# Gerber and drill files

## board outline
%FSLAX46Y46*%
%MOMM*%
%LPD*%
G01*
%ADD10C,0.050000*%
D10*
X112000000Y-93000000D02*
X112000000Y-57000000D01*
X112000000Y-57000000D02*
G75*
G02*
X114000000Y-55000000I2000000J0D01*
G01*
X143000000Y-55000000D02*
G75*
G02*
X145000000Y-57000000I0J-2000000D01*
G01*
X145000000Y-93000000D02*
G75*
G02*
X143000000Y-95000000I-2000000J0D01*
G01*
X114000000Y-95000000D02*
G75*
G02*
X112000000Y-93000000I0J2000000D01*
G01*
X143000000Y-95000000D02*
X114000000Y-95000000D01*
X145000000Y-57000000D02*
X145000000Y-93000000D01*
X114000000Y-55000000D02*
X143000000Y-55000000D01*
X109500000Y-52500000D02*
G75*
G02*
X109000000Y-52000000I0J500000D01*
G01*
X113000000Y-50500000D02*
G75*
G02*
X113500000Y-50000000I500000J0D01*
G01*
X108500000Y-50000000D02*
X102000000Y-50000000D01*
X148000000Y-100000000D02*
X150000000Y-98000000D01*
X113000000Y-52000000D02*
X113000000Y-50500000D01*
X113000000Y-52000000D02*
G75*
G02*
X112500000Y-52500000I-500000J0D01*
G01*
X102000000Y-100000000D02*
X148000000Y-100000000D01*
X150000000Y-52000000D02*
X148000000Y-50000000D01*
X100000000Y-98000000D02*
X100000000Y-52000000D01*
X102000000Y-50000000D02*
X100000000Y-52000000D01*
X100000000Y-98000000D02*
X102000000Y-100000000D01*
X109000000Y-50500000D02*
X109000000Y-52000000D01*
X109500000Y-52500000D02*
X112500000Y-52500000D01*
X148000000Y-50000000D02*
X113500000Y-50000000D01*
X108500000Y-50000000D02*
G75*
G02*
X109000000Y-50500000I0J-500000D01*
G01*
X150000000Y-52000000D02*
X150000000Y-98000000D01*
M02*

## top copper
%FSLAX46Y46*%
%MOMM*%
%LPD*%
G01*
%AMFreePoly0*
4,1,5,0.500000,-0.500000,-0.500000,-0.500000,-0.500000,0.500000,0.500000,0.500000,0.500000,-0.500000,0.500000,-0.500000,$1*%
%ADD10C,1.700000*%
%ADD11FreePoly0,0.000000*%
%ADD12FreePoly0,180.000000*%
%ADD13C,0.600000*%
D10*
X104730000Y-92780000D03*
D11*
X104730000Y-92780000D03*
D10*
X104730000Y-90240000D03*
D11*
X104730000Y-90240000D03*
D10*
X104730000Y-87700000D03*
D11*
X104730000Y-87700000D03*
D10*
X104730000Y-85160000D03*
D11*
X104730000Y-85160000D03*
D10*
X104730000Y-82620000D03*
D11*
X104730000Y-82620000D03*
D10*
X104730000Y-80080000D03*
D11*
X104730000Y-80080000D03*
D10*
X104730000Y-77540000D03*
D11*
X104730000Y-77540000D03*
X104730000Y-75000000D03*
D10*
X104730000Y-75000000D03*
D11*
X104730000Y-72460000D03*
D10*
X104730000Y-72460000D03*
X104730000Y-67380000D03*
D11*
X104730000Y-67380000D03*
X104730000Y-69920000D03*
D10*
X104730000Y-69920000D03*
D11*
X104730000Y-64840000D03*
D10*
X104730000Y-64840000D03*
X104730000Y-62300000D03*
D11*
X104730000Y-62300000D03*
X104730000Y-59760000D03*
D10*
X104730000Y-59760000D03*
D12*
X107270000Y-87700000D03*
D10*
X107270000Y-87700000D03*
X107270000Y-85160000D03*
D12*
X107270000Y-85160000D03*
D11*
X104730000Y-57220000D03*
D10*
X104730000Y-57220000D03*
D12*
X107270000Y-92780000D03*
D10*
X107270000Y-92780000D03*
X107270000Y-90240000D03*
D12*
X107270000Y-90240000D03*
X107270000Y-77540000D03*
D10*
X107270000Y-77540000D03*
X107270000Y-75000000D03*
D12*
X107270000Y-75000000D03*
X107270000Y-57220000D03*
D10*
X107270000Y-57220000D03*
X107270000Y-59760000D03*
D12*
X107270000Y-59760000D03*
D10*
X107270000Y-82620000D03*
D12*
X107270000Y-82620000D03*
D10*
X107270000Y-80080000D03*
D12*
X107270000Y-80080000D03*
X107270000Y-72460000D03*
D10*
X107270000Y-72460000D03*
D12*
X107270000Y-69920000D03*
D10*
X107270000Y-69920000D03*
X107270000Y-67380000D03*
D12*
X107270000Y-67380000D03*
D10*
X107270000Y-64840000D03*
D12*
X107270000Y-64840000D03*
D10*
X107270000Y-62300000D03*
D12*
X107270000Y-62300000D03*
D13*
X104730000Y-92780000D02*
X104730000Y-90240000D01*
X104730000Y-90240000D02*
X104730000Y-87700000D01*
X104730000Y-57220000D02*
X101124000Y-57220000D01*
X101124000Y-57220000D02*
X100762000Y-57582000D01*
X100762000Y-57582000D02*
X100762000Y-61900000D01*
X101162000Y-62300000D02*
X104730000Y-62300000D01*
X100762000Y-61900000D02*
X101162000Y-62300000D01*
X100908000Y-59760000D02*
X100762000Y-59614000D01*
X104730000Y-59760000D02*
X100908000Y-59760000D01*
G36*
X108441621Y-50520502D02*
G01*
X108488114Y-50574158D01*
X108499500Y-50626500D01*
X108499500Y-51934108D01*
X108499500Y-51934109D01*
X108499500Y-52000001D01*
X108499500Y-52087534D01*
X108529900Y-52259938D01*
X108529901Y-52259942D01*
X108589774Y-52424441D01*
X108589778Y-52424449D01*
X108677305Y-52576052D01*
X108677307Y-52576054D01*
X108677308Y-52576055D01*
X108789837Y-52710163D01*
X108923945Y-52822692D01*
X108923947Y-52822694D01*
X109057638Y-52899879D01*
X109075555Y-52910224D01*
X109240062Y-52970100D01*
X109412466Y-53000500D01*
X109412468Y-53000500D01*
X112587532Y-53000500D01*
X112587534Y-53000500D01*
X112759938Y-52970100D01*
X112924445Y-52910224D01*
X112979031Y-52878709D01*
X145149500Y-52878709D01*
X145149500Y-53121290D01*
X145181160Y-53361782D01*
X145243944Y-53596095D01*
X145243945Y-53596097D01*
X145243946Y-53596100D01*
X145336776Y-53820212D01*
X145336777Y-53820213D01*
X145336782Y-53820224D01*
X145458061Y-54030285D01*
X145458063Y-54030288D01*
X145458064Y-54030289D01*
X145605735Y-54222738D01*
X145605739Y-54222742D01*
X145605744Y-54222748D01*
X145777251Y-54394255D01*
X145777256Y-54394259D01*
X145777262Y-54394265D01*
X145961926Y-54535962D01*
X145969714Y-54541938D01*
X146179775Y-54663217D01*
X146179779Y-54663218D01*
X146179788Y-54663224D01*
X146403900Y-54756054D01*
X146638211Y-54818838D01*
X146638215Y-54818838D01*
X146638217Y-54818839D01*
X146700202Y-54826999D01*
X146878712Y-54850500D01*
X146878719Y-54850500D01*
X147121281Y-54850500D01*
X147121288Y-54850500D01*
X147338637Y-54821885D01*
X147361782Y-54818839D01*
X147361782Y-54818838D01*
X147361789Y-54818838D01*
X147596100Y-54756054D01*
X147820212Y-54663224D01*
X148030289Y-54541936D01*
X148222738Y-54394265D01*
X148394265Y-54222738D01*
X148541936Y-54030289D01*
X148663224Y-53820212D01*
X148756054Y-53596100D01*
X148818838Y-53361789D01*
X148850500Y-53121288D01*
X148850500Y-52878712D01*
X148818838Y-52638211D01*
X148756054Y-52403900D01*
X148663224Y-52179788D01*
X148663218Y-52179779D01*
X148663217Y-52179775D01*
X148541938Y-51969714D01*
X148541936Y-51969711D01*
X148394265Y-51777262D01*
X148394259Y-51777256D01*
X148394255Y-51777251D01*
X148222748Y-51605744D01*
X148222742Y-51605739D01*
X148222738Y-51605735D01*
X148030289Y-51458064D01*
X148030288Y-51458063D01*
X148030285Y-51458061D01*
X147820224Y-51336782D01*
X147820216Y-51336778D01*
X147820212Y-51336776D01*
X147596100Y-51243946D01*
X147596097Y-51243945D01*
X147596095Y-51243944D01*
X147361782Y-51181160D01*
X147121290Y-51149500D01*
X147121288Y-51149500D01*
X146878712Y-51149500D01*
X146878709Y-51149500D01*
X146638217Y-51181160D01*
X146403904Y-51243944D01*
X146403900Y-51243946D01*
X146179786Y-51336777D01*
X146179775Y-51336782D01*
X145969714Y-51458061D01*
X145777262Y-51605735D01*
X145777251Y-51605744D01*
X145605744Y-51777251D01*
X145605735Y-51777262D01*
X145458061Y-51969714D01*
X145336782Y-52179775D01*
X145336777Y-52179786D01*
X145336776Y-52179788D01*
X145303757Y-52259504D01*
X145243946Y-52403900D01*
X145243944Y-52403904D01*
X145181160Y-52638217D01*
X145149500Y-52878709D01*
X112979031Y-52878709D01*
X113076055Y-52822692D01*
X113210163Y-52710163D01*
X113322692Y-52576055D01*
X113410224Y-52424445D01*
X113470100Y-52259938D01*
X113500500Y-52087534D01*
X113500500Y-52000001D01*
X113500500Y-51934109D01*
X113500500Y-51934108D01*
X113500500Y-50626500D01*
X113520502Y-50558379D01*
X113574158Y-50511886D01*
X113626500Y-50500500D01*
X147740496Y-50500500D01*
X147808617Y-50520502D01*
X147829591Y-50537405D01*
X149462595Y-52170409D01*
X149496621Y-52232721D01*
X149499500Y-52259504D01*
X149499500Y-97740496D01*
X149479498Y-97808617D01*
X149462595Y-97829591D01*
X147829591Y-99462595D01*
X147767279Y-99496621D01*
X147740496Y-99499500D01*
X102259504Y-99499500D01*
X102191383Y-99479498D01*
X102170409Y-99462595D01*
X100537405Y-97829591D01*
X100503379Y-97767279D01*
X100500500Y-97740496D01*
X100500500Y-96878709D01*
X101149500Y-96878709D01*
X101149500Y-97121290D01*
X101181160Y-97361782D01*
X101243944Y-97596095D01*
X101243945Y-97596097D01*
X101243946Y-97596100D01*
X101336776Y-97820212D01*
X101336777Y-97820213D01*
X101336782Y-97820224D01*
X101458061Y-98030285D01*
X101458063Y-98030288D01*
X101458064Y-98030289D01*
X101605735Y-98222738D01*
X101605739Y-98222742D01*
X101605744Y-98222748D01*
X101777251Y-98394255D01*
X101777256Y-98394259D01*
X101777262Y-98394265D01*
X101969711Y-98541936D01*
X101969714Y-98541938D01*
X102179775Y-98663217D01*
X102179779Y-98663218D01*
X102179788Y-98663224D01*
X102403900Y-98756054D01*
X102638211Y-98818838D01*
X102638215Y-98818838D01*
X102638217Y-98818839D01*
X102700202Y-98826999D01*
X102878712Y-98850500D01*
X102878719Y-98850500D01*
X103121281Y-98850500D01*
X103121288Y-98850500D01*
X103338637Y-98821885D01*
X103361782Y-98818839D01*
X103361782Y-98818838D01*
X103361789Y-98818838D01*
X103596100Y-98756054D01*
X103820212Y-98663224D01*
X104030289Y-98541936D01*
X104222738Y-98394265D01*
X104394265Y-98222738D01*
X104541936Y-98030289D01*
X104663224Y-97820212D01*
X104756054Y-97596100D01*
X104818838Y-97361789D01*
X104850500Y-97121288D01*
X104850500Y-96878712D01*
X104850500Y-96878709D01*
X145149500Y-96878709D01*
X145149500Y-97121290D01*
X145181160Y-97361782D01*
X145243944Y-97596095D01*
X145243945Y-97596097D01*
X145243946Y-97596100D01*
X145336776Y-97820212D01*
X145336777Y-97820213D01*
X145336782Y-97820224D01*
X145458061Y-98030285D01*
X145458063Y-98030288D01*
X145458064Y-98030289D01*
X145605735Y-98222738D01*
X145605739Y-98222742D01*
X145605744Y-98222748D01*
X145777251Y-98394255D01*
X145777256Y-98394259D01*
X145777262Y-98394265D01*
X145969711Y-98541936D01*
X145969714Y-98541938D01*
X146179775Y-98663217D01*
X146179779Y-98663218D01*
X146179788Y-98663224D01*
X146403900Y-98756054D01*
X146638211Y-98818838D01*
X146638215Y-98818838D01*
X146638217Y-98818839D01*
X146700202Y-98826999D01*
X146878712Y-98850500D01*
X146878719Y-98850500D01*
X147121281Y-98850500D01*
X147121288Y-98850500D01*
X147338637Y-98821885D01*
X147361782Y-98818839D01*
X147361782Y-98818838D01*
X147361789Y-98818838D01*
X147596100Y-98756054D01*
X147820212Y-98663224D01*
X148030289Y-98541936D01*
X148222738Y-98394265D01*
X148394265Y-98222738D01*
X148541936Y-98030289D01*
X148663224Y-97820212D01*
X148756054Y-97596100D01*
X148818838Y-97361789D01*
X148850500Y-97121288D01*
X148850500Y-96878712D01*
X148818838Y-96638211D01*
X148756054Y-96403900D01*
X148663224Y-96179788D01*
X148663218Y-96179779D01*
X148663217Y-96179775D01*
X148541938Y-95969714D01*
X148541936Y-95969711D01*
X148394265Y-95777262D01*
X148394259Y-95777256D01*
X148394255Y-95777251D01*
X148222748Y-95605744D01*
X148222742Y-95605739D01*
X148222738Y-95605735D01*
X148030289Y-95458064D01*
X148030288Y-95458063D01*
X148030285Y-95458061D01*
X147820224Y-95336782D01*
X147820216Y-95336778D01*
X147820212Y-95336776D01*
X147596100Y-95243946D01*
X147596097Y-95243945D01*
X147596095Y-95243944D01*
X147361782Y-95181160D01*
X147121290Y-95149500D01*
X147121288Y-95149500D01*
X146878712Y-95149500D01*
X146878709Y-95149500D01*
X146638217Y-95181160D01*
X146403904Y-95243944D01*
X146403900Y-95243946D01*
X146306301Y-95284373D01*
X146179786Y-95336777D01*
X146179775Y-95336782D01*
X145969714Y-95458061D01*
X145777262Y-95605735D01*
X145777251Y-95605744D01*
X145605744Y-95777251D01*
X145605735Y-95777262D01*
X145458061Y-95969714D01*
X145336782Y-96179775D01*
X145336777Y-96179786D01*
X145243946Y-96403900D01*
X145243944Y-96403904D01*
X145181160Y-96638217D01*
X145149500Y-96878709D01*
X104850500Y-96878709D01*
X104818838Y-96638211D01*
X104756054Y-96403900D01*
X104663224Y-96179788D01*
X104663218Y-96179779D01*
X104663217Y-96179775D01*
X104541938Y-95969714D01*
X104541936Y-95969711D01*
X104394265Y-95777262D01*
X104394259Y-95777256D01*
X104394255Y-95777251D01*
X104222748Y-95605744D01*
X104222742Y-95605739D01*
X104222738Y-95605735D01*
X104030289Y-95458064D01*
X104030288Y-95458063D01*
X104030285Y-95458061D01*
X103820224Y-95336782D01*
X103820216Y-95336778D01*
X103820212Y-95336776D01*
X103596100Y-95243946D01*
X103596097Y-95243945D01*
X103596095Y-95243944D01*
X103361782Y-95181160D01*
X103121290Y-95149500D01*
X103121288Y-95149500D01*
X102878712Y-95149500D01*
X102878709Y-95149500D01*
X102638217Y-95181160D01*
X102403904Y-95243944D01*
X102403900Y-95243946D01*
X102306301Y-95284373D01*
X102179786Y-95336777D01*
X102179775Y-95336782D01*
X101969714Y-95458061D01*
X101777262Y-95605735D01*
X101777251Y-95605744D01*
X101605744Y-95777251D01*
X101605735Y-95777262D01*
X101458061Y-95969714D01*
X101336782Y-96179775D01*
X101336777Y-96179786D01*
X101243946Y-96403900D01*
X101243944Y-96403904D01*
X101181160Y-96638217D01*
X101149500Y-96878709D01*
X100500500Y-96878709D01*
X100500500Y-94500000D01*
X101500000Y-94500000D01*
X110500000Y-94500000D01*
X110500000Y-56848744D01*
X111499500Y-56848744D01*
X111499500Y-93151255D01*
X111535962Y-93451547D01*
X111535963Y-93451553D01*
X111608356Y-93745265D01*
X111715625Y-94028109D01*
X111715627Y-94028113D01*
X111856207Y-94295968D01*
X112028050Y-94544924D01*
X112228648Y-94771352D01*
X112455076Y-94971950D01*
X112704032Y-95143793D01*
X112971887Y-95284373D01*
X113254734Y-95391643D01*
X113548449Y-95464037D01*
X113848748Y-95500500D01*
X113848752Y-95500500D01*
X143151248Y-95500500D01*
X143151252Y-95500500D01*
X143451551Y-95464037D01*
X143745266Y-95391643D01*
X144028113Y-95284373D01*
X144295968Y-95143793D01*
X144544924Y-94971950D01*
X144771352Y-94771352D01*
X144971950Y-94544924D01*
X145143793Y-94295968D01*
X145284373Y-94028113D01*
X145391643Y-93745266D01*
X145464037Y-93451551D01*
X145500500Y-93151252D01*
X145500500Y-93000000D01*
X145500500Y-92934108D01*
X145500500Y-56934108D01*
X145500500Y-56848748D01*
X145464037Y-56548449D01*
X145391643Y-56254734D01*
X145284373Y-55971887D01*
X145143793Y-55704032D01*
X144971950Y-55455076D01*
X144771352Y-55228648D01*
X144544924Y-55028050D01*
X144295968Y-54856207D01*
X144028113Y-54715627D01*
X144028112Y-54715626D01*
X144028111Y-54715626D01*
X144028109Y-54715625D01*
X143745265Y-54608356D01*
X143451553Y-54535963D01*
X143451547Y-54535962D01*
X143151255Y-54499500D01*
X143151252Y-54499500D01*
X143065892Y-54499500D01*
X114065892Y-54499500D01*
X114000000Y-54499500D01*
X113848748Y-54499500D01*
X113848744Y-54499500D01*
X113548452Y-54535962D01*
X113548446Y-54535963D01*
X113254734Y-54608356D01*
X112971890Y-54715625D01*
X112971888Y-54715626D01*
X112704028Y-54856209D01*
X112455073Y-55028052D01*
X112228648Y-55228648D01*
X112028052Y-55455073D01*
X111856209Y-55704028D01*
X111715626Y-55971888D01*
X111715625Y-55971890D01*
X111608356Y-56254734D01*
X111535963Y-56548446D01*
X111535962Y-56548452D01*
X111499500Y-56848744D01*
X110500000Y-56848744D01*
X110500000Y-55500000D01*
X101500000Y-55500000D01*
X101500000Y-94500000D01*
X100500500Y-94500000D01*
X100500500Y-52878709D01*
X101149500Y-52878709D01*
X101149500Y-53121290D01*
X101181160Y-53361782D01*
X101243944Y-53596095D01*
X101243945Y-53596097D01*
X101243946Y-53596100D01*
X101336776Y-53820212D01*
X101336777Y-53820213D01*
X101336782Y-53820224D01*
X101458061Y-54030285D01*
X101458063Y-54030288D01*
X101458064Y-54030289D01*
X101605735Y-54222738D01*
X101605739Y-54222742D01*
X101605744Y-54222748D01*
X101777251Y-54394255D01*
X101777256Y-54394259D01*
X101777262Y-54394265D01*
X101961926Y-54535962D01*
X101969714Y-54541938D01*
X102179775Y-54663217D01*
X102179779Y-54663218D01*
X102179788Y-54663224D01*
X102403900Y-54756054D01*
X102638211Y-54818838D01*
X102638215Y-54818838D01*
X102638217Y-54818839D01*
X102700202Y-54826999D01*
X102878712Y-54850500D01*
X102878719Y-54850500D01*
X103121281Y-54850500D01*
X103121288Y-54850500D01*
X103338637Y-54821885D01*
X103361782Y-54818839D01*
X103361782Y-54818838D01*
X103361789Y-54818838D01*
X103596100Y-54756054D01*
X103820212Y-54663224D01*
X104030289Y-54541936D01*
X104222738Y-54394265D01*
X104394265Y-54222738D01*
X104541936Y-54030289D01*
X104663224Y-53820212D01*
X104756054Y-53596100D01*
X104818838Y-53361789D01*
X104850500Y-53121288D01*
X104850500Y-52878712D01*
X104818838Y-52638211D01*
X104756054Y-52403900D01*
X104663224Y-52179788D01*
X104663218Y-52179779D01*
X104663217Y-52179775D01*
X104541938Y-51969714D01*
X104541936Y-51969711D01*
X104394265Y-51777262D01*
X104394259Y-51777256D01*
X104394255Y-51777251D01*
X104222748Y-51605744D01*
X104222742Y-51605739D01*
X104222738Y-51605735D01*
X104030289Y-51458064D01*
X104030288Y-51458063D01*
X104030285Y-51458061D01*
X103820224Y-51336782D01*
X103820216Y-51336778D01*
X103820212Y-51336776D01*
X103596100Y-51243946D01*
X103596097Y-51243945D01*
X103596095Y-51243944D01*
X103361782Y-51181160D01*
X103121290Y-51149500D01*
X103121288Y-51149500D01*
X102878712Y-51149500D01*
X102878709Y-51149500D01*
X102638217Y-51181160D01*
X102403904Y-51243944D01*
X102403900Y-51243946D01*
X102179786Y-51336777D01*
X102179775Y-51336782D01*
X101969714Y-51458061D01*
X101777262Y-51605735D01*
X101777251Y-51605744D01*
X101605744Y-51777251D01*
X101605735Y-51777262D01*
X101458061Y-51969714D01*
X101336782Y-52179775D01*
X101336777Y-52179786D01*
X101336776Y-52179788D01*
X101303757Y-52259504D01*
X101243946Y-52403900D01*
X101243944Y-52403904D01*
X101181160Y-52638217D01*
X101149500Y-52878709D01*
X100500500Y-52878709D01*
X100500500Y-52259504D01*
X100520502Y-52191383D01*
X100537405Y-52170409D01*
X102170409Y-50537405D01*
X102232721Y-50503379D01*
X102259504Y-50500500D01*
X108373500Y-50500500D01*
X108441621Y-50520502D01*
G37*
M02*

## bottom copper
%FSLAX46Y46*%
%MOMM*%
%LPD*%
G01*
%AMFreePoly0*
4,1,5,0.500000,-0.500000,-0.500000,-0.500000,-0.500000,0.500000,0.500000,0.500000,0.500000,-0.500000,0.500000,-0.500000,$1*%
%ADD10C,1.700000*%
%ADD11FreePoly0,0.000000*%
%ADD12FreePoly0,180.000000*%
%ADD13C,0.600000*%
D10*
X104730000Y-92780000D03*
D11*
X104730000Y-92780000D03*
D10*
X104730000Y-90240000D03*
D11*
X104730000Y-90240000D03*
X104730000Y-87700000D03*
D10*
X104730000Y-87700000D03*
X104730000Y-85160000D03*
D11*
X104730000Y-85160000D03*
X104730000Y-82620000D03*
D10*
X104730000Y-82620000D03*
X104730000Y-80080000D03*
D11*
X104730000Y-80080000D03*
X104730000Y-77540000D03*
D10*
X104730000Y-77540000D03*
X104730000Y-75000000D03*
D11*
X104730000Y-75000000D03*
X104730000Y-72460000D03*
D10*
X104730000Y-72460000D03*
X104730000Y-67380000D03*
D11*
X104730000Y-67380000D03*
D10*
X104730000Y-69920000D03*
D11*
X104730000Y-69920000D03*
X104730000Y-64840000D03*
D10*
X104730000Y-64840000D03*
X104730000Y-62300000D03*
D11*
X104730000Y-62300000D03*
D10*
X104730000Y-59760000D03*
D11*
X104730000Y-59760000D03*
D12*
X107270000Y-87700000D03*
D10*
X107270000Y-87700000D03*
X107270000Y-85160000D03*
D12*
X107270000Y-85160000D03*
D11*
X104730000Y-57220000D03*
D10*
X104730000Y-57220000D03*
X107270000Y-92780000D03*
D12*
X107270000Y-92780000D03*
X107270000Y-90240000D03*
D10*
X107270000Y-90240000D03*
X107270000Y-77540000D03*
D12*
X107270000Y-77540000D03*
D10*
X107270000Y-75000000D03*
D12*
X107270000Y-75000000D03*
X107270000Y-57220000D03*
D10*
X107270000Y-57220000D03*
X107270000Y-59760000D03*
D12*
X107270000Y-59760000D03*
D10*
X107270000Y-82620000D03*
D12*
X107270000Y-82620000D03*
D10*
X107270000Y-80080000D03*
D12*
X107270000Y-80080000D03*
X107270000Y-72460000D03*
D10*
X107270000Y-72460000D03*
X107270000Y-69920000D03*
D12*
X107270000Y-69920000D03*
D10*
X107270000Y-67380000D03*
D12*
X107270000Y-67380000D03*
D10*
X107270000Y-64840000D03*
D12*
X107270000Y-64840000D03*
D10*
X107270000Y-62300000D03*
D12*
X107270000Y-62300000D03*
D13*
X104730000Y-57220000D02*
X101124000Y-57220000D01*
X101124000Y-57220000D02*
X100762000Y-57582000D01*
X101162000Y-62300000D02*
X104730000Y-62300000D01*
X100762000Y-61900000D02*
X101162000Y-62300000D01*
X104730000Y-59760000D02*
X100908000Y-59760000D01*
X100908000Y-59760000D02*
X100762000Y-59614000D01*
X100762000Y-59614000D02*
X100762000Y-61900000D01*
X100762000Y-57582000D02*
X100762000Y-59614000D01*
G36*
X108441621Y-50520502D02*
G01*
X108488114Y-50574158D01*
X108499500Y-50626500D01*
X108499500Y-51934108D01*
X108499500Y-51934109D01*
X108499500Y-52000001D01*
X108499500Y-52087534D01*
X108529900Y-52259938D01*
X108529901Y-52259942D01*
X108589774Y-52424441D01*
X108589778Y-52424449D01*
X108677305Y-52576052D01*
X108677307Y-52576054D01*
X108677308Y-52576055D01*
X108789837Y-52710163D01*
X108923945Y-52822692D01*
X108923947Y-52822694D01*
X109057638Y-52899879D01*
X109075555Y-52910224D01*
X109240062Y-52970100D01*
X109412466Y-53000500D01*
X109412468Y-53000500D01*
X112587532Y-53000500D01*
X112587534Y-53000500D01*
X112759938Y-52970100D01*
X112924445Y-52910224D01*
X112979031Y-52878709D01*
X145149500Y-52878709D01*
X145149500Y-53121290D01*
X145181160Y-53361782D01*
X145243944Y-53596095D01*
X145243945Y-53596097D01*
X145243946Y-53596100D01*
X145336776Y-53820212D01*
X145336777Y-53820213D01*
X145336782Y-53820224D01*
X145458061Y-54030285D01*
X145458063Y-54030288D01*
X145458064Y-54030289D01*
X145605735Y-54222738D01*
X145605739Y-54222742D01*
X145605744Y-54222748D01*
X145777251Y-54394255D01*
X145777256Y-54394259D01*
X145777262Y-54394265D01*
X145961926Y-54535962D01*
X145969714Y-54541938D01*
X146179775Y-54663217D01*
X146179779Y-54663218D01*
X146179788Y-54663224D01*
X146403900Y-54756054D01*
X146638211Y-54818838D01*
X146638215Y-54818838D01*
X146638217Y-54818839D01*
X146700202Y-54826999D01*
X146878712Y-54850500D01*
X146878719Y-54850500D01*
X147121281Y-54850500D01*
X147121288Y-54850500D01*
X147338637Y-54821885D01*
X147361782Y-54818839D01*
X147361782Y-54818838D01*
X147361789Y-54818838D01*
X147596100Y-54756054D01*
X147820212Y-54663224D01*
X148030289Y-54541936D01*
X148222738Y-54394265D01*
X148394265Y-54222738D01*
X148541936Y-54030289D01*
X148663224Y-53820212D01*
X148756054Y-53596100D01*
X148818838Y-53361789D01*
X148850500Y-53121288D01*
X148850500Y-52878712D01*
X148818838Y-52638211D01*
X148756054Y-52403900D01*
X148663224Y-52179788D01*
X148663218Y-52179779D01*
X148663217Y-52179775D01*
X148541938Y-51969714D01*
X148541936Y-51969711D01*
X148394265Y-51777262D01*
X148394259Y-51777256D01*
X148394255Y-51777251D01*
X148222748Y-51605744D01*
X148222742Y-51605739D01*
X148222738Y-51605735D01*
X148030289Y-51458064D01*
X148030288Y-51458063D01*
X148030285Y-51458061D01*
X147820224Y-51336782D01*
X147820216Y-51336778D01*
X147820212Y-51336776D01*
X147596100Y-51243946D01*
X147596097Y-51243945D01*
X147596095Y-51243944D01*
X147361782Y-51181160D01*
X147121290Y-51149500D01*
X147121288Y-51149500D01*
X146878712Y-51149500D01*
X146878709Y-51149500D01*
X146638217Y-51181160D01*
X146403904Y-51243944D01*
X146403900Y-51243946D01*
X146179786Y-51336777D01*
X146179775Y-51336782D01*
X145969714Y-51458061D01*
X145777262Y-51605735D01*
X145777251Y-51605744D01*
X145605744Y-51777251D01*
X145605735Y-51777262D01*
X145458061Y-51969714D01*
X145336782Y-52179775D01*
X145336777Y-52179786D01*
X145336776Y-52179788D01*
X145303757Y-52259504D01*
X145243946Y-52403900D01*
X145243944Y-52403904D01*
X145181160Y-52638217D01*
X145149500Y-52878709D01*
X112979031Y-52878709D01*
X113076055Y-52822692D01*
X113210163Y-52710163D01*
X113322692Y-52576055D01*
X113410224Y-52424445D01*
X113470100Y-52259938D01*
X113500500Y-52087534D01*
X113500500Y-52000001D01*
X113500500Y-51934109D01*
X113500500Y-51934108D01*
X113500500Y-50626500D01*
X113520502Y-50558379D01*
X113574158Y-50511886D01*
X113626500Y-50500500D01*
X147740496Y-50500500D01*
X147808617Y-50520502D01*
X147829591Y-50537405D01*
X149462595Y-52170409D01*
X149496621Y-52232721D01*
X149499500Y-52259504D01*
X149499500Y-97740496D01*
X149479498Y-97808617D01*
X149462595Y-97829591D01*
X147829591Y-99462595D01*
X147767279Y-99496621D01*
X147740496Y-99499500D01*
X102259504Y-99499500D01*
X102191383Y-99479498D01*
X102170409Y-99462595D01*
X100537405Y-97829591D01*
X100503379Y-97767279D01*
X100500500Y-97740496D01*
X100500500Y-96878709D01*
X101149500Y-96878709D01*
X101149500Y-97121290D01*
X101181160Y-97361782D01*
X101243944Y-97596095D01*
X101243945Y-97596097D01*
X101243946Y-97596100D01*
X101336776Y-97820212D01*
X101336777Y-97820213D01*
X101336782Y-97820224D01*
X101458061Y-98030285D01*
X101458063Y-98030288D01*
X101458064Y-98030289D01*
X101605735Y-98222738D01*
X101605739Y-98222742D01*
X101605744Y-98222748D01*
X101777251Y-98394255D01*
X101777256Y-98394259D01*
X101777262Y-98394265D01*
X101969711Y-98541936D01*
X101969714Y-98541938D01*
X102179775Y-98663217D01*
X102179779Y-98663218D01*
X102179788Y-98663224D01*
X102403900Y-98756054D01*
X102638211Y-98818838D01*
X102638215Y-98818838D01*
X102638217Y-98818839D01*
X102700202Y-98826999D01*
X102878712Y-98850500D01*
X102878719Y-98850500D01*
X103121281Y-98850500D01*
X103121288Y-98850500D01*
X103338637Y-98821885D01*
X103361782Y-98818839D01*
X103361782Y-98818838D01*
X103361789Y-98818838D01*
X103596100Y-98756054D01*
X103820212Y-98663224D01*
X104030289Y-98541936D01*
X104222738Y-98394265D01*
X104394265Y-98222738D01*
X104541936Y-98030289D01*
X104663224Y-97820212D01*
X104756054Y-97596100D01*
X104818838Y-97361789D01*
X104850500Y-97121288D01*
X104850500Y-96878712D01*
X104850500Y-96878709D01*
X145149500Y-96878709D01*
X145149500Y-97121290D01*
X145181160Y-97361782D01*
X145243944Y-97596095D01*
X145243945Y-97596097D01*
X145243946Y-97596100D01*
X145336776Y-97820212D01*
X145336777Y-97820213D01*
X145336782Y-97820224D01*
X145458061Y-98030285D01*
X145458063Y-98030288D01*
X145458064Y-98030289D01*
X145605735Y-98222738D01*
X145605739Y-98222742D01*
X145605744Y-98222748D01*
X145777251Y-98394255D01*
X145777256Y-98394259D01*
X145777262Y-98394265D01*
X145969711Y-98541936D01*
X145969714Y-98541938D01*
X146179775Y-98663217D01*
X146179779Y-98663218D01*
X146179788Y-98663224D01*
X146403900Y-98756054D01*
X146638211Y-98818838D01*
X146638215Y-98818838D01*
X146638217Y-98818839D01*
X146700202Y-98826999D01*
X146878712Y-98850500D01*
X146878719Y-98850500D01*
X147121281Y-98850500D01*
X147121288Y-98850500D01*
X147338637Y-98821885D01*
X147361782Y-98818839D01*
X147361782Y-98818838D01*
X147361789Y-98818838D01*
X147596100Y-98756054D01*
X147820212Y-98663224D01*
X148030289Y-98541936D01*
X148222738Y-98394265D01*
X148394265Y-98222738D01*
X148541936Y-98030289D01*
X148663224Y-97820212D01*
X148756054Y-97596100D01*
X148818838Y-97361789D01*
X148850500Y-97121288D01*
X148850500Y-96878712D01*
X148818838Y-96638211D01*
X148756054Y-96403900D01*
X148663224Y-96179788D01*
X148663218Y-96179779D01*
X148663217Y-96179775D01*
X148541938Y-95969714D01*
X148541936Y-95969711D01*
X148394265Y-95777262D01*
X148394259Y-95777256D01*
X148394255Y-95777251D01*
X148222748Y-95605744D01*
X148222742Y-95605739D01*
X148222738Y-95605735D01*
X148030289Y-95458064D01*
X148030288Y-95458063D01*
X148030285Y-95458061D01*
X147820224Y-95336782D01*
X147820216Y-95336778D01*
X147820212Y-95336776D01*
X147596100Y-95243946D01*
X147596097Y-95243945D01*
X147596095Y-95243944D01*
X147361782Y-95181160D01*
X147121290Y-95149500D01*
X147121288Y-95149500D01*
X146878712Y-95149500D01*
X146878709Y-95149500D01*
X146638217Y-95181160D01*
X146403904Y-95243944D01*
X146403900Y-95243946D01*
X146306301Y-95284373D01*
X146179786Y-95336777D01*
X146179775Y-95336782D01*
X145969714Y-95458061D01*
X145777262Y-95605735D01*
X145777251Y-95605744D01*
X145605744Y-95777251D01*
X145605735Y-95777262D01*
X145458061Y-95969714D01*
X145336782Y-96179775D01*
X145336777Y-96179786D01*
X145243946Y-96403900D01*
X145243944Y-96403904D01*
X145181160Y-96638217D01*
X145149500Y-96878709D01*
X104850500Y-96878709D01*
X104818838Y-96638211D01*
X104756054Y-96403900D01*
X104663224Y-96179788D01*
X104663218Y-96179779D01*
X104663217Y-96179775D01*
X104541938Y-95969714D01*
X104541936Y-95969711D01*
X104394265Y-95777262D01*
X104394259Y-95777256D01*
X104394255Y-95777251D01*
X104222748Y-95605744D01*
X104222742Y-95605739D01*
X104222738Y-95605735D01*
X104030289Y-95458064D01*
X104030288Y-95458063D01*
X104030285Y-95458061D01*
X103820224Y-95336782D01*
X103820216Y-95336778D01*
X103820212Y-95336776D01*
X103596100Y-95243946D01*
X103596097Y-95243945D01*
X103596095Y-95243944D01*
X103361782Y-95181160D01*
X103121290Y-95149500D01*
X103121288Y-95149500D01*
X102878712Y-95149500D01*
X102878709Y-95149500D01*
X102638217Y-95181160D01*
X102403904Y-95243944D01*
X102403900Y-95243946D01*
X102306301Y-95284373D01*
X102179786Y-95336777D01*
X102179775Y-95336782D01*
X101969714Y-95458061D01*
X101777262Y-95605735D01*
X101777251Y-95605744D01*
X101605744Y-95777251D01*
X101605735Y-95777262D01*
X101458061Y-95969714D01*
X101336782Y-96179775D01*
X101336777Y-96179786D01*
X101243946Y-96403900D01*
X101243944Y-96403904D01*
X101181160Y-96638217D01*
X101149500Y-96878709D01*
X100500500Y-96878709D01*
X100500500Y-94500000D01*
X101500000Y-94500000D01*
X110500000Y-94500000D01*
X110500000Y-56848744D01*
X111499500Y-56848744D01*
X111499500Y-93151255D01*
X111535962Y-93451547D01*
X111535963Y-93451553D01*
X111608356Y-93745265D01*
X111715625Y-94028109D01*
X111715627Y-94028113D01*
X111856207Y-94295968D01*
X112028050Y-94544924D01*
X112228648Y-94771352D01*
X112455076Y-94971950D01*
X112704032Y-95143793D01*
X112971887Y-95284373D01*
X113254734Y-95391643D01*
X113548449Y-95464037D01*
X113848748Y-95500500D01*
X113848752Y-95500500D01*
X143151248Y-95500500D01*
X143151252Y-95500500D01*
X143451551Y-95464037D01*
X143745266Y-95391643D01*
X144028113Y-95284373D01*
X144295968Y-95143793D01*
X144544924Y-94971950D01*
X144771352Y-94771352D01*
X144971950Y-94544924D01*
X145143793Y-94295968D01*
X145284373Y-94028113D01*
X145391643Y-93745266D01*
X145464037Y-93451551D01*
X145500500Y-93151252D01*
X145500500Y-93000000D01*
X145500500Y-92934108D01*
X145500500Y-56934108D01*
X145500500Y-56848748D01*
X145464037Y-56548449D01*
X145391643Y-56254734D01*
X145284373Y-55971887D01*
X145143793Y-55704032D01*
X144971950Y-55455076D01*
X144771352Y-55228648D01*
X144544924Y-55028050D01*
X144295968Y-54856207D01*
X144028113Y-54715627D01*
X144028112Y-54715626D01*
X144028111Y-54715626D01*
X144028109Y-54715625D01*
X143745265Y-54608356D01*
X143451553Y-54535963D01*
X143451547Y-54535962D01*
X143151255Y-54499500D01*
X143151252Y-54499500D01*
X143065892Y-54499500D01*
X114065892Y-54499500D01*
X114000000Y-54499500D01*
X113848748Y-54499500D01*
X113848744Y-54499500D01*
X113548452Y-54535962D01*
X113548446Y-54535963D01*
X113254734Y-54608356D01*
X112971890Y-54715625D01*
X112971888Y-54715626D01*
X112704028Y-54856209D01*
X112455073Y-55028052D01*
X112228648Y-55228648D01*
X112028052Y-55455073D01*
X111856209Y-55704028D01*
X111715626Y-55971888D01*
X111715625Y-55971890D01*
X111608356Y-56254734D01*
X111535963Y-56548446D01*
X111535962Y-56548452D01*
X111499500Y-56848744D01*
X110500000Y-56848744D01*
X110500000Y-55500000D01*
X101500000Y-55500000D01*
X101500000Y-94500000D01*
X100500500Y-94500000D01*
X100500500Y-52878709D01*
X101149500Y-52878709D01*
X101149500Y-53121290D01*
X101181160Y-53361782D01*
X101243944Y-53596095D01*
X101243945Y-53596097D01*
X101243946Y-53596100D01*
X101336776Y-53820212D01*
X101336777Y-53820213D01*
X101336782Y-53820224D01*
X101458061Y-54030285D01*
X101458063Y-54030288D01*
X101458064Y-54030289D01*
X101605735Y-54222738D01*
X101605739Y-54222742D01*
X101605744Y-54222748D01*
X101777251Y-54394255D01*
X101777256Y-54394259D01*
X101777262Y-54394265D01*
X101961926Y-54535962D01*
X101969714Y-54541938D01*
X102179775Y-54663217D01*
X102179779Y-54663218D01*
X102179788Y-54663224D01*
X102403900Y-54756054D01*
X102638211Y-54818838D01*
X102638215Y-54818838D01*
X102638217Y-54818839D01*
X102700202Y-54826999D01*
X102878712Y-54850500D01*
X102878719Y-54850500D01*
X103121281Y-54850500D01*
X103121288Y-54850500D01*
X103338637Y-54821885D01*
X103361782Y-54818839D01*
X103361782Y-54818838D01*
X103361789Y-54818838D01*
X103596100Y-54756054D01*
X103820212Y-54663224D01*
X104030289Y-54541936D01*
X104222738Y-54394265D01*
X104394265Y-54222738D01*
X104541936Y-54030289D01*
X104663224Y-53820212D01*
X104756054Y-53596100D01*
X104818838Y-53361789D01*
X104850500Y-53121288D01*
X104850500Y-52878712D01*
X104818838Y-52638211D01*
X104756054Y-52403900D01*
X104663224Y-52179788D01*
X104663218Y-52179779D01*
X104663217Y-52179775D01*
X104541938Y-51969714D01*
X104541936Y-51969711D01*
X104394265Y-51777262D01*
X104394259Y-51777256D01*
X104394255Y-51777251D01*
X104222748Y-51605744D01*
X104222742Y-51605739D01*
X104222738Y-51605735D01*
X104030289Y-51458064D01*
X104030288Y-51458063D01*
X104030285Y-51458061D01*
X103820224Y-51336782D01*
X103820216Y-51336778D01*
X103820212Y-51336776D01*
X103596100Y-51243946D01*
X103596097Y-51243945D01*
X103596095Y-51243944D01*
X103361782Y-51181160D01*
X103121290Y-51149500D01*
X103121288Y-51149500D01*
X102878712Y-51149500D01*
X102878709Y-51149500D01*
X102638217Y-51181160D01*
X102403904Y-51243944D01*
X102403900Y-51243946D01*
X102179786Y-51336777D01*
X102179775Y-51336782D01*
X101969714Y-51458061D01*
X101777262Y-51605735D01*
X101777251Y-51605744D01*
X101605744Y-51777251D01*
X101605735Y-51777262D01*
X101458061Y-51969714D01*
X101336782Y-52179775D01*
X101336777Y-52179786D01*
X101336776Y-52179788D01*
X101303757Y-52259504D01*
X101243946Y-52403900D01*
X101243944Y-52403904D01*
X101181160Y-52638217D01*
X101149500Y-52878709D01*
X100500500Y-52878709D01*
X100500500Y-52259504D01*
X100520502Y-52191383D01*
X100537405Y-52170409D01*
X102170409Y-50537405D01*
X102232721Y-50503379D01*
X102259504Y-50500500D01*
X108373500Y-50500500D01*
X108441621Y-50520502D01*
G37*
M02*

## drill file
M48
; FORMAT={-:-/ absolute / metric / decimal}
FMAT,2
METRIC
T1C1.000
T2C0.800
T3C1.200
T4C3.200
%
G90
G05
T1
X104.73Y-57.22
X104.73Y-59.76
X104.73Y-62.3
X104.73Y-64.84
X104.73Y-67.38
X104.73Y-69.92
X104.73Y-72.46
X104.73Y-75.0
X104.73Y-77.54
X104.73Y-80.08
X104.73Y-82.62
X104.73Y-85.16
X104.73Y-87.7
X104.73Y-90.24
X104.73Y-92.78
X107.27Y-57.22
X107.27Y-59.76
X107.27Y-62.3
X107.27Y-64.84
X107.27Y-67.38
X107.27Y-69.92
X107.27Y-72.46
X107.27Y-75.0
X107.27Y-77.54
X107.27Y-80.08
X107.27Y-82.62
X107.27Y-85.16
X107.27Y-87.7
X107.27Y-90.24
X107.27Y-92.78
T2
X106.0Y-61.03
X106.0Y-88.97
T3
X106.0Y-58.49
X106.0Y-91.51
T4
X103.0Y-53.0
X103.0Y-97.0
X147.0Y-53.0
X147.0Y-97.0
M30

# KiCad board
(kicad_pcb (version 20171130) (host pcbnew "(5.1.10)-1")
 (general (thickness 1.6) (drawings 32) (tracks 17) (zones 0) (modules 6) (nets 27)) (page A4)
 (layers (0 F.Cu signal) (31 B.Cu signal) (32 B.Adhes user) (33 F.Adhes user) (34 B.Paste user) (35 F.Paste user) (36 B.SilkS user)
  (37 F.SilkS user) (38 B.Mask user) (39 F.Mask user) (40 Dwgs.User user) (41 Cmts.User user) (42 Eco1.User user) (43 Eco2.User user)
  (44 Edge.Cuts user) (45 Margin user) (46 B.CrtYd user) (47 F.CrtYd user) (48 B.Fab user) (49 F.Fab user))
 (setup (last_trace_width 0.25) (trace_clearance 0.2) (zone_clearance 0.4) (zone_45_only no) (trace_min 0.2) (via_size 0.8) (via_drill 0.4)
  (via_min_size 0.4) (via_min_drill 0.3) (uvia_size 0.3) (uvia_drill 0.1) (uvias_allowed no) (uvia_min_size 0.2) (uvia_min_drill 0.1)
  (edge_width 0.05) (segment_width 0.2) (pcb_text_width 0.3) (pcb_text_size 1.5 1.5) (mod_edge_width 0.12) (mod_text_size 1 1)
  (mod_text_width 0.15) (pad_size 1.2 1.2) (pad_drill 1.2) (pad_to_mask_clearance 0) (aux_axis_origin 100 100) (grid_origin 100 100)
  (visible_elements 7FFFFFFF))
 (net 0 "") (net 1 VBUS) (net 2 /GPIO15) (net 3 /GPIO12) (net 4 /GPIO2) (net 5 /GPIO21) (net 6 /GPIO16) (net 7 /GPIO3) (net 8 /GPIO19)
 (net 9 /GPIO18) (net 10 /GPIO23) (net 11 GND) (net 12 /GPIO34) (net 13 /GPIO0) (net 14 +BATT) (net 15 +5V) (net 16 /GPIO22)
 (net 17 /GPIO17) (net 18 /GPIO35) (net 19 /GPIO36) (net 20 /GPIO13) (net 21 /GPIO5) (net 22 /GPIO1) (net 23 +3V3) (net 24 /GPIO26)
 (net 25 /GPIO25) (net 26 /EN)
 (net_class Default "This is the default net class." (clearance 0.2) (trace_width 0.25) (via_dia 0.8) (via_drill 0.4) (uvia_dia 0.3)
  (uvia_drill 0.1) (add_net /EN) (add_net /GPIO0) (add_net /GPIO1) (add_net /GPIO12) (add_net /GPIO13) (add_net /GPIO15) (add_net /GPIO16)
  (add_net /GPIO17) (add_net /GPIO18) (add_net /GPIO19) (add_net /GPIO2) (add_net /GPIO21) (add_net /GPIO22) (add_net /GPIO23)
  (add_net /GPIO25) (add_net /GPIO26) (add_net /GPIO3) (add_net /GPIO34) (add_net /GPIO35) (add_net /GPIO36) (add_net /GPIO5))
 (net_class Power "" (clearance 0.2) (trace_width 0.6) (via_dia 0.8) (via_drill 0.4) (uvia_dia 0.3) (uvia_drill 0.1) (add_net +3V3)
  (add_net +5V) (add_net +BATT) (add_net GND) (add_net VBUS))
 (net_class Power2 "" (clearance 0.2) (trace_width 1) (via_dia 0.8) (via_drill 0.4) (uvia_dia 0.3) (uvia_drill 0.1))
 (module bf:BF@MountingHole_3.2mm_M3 (layer F.Cu) (at 147 97)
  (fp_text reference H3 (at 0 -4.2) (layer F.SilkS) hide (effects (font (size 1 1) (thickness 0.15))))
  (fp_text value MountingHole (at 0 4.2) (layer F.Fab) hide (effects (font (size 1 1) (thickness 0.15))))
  (pad "" np_thru_hole circle (at 0 0) (size 3.2 3.2) (drill 3.2) (layers *.Cu *.Mask)))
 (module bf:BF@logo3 (layer F.Cu) (at 130 97.5)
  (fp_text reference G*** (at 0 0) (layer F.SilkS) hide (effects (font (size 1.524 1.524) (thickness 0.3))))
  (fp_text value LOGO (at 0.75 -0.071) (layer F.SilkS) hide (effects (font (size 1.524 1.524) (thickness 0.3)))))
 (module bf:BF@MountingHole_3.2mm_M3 (layer F.Cu) (at 103 97)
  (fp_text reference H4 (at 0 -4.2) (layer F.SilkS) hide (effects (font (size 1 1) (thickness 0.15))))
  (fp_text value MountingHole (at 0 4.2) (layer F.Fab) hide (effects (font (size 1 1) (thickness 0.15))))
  (pad "" np_thru_hole circle (at 0 0) (size 3.2 3.2) (drill 3.2) (layers *.Cu *.Mask)))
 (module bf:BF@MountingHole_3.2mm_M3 (layer F.Cu) (at 147 53)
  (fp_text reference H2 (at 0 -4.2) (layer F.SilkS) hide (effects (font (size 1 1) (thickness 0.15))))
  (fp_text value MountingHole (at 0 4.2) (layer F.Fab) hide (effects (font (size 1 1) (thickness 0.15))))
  (pad "" np_thru_hole circle (at 0 0) (size 3.2 3.2) (drill 3.2) (layers *.Cu *.Mask)))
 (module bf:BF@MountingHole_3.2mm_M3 (layer F.Cu) (at 103 53)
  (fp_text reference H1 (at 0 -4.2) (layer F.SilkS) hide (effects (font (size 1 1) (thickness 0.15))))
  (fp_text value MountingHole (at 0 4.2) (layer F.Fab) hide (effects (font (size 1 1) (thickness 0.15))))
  (pad "" np_thru_hole circle (at 0 0) (size 3.2 3.2) (drill 3.2) (layers *.Cu *.Mask)))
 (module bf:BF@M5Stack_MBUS (layer F.Cu) (at 106 75)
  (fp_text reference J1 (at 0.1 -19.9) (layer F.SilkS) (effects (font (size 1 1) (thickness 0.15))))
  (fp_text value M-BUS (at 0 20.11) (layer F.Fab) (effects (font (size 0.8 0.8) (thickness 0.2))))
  (pad 30 thru_hole circle (at -1.27 17.78) (size 1.7 1.7) (drill 1) (layers *.Cu *.Mask) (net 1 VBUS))
  (pad 30 smd custom (at -1.27 17.78) (size 1 1) (layers B.Cu B.Mask) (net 1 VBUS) (zone_connect 0)
   (options (clearance outline) (anchor rect)) (primitives))
  (pad 30 smd custom (at -1.27 17.78) (size 1 1) (layers F.Cu F.Mask) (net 1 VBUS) (zone_connect 0)
   (options (clearance outline) (anchor rect)) (primitives))
  (pad 28 thru_hole circle (at -1.27 15.24) (size 1.7 1.7) (drill 1) (layers *.Cu *.Mask) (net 1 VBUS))
  (pad 28 smd custom (at -1.27 15.24) (size 1 1) (layers B.Cu B.Mask) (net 1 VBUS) (zone_connect 0)
   (options (clearance outline) (anchor rect)) (primitives))
  (pad 28 smd custom (at -1.27 15.24) (size 1 1) (layers F.Cu F.Mask) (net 1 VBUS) (zone_connect 0)
   (options (clearance outline) (anchor rect)) (primitives))
  (pad 26 smd custom (at -1.27 12.7) (size 1 1) (layers B.Cu B.Mask) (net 1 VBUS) (zone_connect 0)
   (options (clearance outline) (anchor rect)) (primitives))
  (pad 26 thru_hole circle (at -1.27 12.7) (size 1.7 1.7) (drill 1) (layers *.Cu *.Mask) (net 1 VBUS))
  (pad 26 smd custom (at -1.27 12.7) (size 1 1) (layers F.Cu F.Mask) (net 1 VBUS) (zone_connect 0)
   (options (clearance outline) (anchor rect)) (primitives))
  (pad 24 thru_hole circle (at -1.27 10.16) (size 1.7 1.7) (drill 1) (layers *.Cu *.Mask) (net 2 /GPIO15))
  (pad 24 smd custom (at -1.27 10.16) (size 1 1) (layers B.Cu B.Mask) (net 2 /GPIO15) (zone_connect 0)
   (options (clearance outline) (anchor rect)) (primitives))
  (pad 24 smd custom (at -1.27 10.16) (size 1 1) (layers F.Cu F.Mask) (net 2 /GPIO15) (zone_connect 0)
   (options (clearance outline) (anchor rect)) (primitives))
  (pad 22 smd custom (at -1.27 7.62) (size 1 1) (layers B.Cu B.Mask) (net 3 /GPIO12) (zone_connect 0)
   (options (clearance outline) (anchor rect)) (primitives))
  (pad 22 thru_hole circle (at -1.27 7.62) (size 1.7 1.7) (drill 1) (layers *.Cu *.Mask) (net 3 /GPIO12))
  (pad 22 smd custom (at -1.27 7.62) (size 1 1) (layers F.Cu F.Mask) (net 3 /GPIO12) (zone_connect 0)
   (options (clearance outline) (anchor rect)) (primitives))
  (pad 20 thru_hole circle (at -1.27 5.08) (size 1.7 1.7) (drill 1) (layers *.Cu *.Mask) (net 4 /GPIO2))
  (pad 20 smd custom (at -1.27 5.08) (size 1 1) (layers F.Cu F.Mask) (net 4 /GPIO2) (zone_connect 0)
   (options (clearance outline) (anchor rect)) (primitives))
  (pad 20 smd custom (at -1.27 5.08) (size 1 1) (layers B.Cu B.Mask) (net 4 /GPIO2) (zone_connect 0)
   (options (clearance outline) (anchor rect)) (primitives))
  (pad 18 smd custom (at -1.27 2.54) (size 1 1) (layers B.Cu B.Mask) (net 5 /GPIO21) (zone_connect 0)
   (options (clearance outline) (anchor rect)) (primitives))
  (pad 18 thru_hole circle (at -1.27 2.54) (size 1.7 1.7) (drill 1) (layers *.Cu *.Mask) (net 5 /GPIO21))
  (pad 18 smd custom (at -1.27 2.54) (size 1 1) (layers F.Cu F.Mask) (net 5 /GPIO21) (zone_connect 0)
   (options (clearance outline) (anchor rect)) (primitives))
  (pad 16 smd custom (at -1.27 0) (size 1 1) (layers F.Cu F.Mask) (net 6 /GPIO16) (zone_connect 0)
   (options (clearance outline) (anchor rect)) (primitives))
  (pad 16 thru_hole circle (at -1.27 0) (size 1.7 1.7) (drill 1) (layers *.Cu *.Mask) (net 6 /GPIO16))
  (pad 16 smd custom (at -1.27 0) (size 1 1) (layers B.Cu B.Mask) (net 6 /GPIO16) (zone_connect 0)
   (options (clearance outline) (anchor rect)) (primitives))
  (pad 14 smd custom (at -1.27 -2.54) (size 1 1) (layers B.Cu B.Mask) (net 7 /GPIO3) (zone_connect 0)
   (options (clearance outline) (anchor rect)) (primitives))
  (pad 14 smd custom (at -1.27 -2.54) (size 1 1) (layers F.Cu F.Mask) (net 7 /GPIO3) (zone_connect 0)
   (options (clearance outline) (anchor rect)) (primitives))
  (pad 14 thru_hole circle (at -1.27 -2.54) (size 1.7 1.7) (drill 1) (layers *.Cu *.Mask) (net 7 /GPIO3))
  (pad 10 thru_hole circle (at -1.27 -7.62) (size 1.7 1.7) (drill 1) (layers *.Cu *.Mask) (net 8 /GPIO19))
  (pad 10 smd custom (at -1.27 -7.62) (size 1 1) (layers B.Cu B.Mask) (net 8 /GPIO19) (zone_connect 0)
   (options (clearance outline) (anchor rect)) (primitives))
  (pad 10 smd custom (at -1.27 -7.62) (size 1 1) (layers F.Cu F.Mask) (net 8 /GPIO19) (zone_connect 0)
   (options (clearance outline) (anchor rect)) (primitives))
  (pad 12 smd custom (at -1.27 -5.08) (size 1 1) (layers F.Cu F.Mask) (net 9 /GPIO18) (zone_connect 0)
   (options (clearance outline) (anchor rect)) (primitives))
  (pad 12 thru_hole circle (at -1.27 -5.08) (size 1.7 1.7) (drill 1) (layers *.Cu *.Mask) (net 9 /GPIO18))
  (pad 12 smd custom (at -1.27 -5.08) (size 1 1) (layers B.Cu B.Mask) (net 9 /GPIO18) (zone_connect 0)
   (options (clearance outline) (anchor rect)) (primitives))
  (pad 8 smd custom (at -1.27 -10.16) (size 1 1) (layers B.Cu B.Mask) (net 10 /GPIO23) (zone_connect 0)
   (options (clearance outline) (anchor rect)) (primitives))
  (pad 8 smd custom (at -1.27 -10.16) (size 1 1) (layers F.Cu F.Mask) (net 10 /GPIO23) (zone_connect 0)
   (options (clearance outline) (anchor rect)) (primitives))
  (pad 8 thru_hole circle (at -1.27 -10.16) (size 1.7 1.7) (drill 1) (layers *.Cu *.Mask) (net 10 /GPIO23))
  (pad 6 thru_hole circle (at -1.27 -12.7) (size 1.7 1.7) (drill 1) (layers *.Cu *.Mask) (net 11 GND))
  (pad 6 smd custom (at -1.27 -12.7) (size 1 1) (layers F.Cu F.Mask) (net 11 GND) (zone_connect 0)
   (options (clearance outline) (anchor rect)) (primitives))
  (pad 6 smd custom (at -1.27 -12.7) (size 1 1) (layers B.Cu B.Mask) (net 11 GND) (zone_connect 0)
   (options (clearance outline) (anchor rect)) (primitives))
  (pad 4 smd custom (at -1.27 -15.24) (size 1 1) (layers F.Cu F.Mask) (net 11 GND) (zone_connect 0)
   (options (clearance outline) (anchor rect)) (primitives))
  (pad 4 thru_hole circle (at -1.27 -15.24) (size 1.7 1.7) (drill 1) (layers *.Cu *.Mask) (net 11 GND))
  (pad 4 smd custom (at -1.27 -15.24) (size 1 1) (layers B.Cu B.Mask) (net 11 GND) (zone_connect 0)
   (options (clearance outline) (anchor rect)) (primitives))
  (pad 25 smd custom (at 1.27 12.7 180) (size 1 1) (layers B.Cu B.Mask) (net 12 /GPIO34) (zone_connect 0)
   (options (clearance outline) (anchor rect)) (primitives))
  (pad 25 smd custom (at 1.27 12.7 180) (size 1 1) (layers F.Cu F.Mask) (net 12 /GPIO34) (zone_connect 0)
   (options (clearance outline) (anchor rect)) (primitives))
  (pad 25 thru_hole circle (at 1.27 12.7 180) (size 1.7 1.7) (drill 1) (layers *.Cu *.Mask) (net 12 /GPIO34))
  (pad 23 thru_hole circle (at 1.27 10.16 180) (size 1.7 1.7) (drill 1) (layers *.Cu *.Mask) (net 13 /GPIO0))
  (pad 23 smd custom (at 1.27 10.16 180) (size 1 1) (layers F.Cu F.Mask) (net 13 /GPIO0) (zone_connect 0)
   (options (clearance outline) (anchor rect)) (primitives))
  (pad 23 smd custom (at 1.27 10.16 180) (size 1 1) (layers B.Cu B.Mask) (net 13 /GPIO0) (zone_connect 0)
   (options (clearance outline) (anchor rect)) (primitives))
  (pad 2 smd custom (at -1.27 -17.78) (size 1 1) (layers F.Cu F.Mask) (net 11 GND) (zone_connect 0)
   (options (clearance outline) (anchor rect)) (primitives))
  (pad 2 smd custom (at -1.27 -17.78) (size 1 1) (layers B.Cu B.Mask) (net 11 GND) (zone_connect 0)
   (options (clearance outline) (anchor rect)) (primitives))
  (pad 2 thru_hole circle (at -1.27 -17.78) (size 1.7 1.7) (drill 1) (layers *.Cu *.Mask) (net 11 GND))
  (pad 29 smd custom (at 1.27 17.78 180) (size 1 1) (layers F.Cu F.Mask) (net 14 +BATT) (zone_connect 0)
   (options (clearance outline) (anchor rect)) (primitives))
  (pad 29 thru_hole circle (at 1.27 17.78 180) (size 1.7 1.7) (drill 1) (layers *.Cu *.Mask) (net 14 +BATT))
  (pad 29 smd custom (at 1.27 17.78 180) (size 1 1) (layers B.Cu B.Mask) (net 14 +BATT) (zone_connect 0)
   (options (clearance outline) (anchor rect)) (primitives))
  (pad 27 smd custom (at 1.27 15.24 180) (size 1 1) (layers B.Cu B.Mask) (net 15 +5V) (zone_connect 0)
   (options (clearance outline) (anchor rect)) (primitives))
  (pad 27 thru_hole circle (at 1.27 15.24 180) (size 1.7 1.7) (drill 1) (layers *.Cu *.Mask) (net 15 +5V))
  (pad 27 smd custom (at 1.27 15.24 180) (size 1 1) (layers F.Cu F.Mask) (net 15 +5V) (zone_connect 0)
   (options (clearance outline) (anchor rect)) (primitives))
  (pad 17 smd custom (at 1.27 2.54 180) (size 1 1) (layers F.Cu F.Mask) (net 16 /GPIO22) (zone_connect 0)
   (options (clearance outline) (anchor rect)) (primitives))
  (pad 17 thru_hole circle (at 1.27 2.54 180) (size 1.7 1.7) (drill 1) (layers *.Cu *.Mask) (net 16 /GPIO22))
  (pad 17 smd custom (at 1.27 2.54 180) (size 1 1) (layers B.Cu B.Mask) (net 16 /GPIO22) (zone_connect 0)
   (options (clearance outline) (anchor rect)) (primitives))
  (pad 15 thru_hole circle (at 1.27 0 180) (size 1.7 1.7) (drill 1) (layers *.Cu *.Mask) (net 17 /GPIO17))
  (pad 15 smd custom (at 1.27 0 180) (size 1 1) (layers B.Cu B.Mask) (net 17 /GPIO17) (zone_connect 0)
   (options (clearance outline) (anchor rect)) (primitives))
  (pad 15 smd custom (at 1.27 0 180) (size 1 1) (layers F.Cu F.Mask) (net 17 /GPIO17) (zone_connect 0)
   (options (clearance outline) (anchor rect)) (primitives))
  (pad "" np_thru_hole circle (at 0 13.97 180) (size 0.8 0.8) (drill 0.8) (layers *.Cu *.Mask))
  (pad 1 smd custom (at 1.27 -17.78 180) (size 1 1) (layers F.Cu F.Mask) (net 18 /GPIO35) (zone_connect 0)
   (options (clearance outline) (anchor rect)) (primitives))
  (pad 1 smd custom (at 1.27 -17.78 180) (size 1 1) (layers B.Cu B.Mask) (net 18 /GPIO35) (zone_connect 0)
   (options (clearance outline) (anchor rect)) (primitives))
  (pad "" np_thru_hole circle (at 0 16.51 180) (size 1.2 1.2) (drill 1.2) (layers *.Cu *.Mask))
  (pad "" np_thru_hole circle (at 0 -13.97 180) (size 0.8 0.8) (drill 0.8) (layers *.Cu *.Mask))
  (pad 1 thru_hole circle (at 1.27 -17.78 180) (size 1.7 1.7) (drill 1) (layers *.Cu *.Mask) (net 18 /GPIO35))
  (pad "" np_thru_hole circle (at 0 -16.51 180) (size 1.2 1.2) (drill 1.2) (layers *.Cu *.Mask))
  (pad 3 thru_hole circle (at 1.27 -15.24 180) (size 1.7 1.7) (drill 1) (layers *.Cu *.Mask) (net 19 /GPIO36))
  (pad 3 smd custom (at 1.27 -15.24 180) (size 1 1) (layers B.Cu B.Mask) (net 19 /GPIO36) (zone_connect 0)
   (options (clearance outline) (anchor rect)) (primitives))
  (pad 3 smd custom (at 1.27 -15.24 180) (size 1 1) (layers F.Cu F.Mask) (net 19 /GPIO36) (zone_connect 0)
   (options (clearance outline) (anchor rect)) (primitives))
  (pad 21 thru_hole circle (at 1.27 7.62 180) (size 1.7 1.7) (drill 1) (layers *.Cu *.Mask) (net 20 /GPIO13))
  (pad 21 smd custom (at 1.27 7.62 180) (size 1 1) (layers B.Cu B.Mask) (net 20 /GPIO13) (zone_connect 0)
   (options (clearance outline) (anchor rect)) (primitives))
  (pad 21 smd custom (at 1.27 7.62 180) (size 1 1) (layers F.Cu F.Mask) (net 20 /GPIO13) (zone_connect 0)
   (options (clearance outline) (anchor rect)) (primitives))
  (pad 19 thru_hole circle (at 1.27 5.08 180) (size 1.7 1.7) (drill 1) (layers *.Cu *.Mask) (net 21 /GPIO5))
  (pad 19 smd custom (at 1.27 5.08 180) (size 1 1) (layers F.Cu F.Mask) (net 21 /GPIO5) (zone_connect 0)
   (options (clearance outline) (anchor rect)) (primitives))
  (pad 19 smd custom (at 1.27 5.08 180) (size 1 1) (layers B.Cu B.Mask) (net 21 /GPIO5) (zone_connect 0)
   (options (clearance outline) (anchor rect)) (primitives))
  (pad 13 smd custom (at 1.27 -2.54 180) (size 1 1) (layers F.Cu F.Mask) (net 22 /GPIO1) (zone_connect 0)
   (options (clearance outline) (anchor rect)) (primitives))
  (pad 13 smd custom (at 1.27 -2.54 180) (size 1 1) (layers B.Cu B.Mask) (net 22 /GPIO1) (zone_connect 0)
   (options (clearance outline) (anchor rect)) (primitives))
  (pad 13 thru_hole circle (at 1.27 -2.54 180) (size 1.7 1.7) (drill 1) (layers *.Cu *.Mask) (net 22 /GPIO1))
  (pad 11 smd custom (at 1.27 -5.08 180) (size 1 1) (layers F.Cu F.Mask) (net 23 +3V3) (zone_connect 0)
   (options (clearance outline) (anchor rect)) (primitives))
  (pad 11 thru_hole circle (at 1.27 -5.08 180) (size 1.7 1.7) (drill 1) (layers *.Cu *.Mask) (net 23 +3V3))
  (pad 11 smd custom (at 1.27 -5.08 180) (size 1 1) (layers B.Cu B.Mask) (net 23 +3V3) (zone_connect 0)
   (options (clearance outline) (anchor rect)) (primitives))
  (pad 9 thru_hole circle (at 1.27 -7.62 180) (size 1.7 1.7) (drill 1) (layers *.Cu *.Mask) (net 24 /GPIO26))
  (pad 9 smd custom (at 1.27 -7.62 180) (size 1 1) (layers B.Cu B.Mask) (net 24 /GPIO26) (zone_connect 0)
   (options (clearance outline) (anchor rect)) (primitives))
  (pad 9 smd custom (at 1.27 -7.62 180) (size 1 1) (layers F.Cu F.Mask) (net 24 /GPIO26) (zone_connect 0)
   (options (clearance outline) (anchor rect)) (primitives))
  (pad 7 thru_hole circle (at 1.27 -10.16 180) (size 1.7 1.7) (drill 1) (layers *.Cu *.Mask) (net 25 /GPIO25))
  (pad 7 smd custom (at 1.27 -10.16 180) (size 1 1) (layers F.Cu F.Mask) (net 25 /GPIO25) (zone_connect 0)
   (options (clearance outline) (anchor rect)) (primitives))
  (pad 7 smd custom (at 1.27 -10.16 180) (size 1 1) (layers B.Cu B.Mask) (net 25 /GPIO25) (zone_connect 0)
   (options (clearance outline) (anchor rect)) (primitives))
  (pad 5 thru_hole circle (at 1.27 -12.7 180) (size 1.7 1.7) (drill 1) (layers *.Cu *.Mask) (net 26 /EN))
  (pad 5 smd custom (at 1.27 -12.7 180) (size 1 1) (layers B.Cu B.Mask) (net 26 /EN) (zone_connect 0)
   (options (clearance outline) (anchor rect)) (primitives))
  (pad 5 smd custom (at 1.27 -12.7 180) (size 1 1) (layers F.Cu F.Mask) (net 26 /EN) (zone_connect 0)
   (options (clearance outline) (anchor rect)) (primitives)))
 (gr_line (start 112 93) (end 112 57) (layer Edge.Cuts) (width 0.05))
 (gr_arc (start 114 57) (end 114 55) (angle -90) (layer Edge.Cuts) (width 0.05))
 (gr_arc (start 143 57) (end 145 57) (angle -90) (layer Edge.Cuts) (width 0.05))
 (gr_arc (start 143 93) (end 143 95) (angle -90) (layer Edge.Cuts) (width 0.05))
 (gr_arc (start 114 93) (end 112 93) (angle -90) (layer Edge.Cuts) (width 0.05))
 (gr_line (start 143 95) (end 114 95) (layer Edge.Cuts) (width 0.05))
 (gr_line (start 145 57) (end 145 93) (layer Edge.Cuts) (width 0.05))
 (gr_line (start 114 55) (end 143 55) (layer Edge.Cuts) (width 0.05))
 (gr_arc (start 109.5 52) (end 109 52) (angle -90) (layer Edge.Cuts) (width 0.05))
 (gr_arc (start 113.5 50.5) (end 113.5 50) (angle -90) (layer Edge.Cuts) (width 0.05))
 (gr_line (start 108.5 50) (end 102 50) (layer Edge.Cuts) (width 0.05))
 (gr_line (start 148 100) (end 150 98) (layer Edge.Cuts) (width 0.05))
 (gr_line (start 113 52) (end 113 50.5) (layer Edge.Cuts) (width 0.05))
 (gr_arc (start 112.5 52) (end 112.5 52.5) (angle -90) (layer Edge.Cuts) (width 0.05))
 (gr_line (start 102 100) (end 148 100) (layer Edge.Cuts) (width 0.05))
 (gr_line (start 150 52) (end 148 50) (layer Edge.Cuts) (width 0.05))
 (gr_line (start 100 98) (end 100 52) (layer Edge.Cuts) (width 0.05))
 (gr_line (start 102 50) (end 100 52) (layer Edge.Cuts) (width 0.05))
 (gr_line (start 100 98) (end 102 100) (layer Edge.Cuts) (width 0.05))
 (gr_line (start 109 50.5) (end 109 52) (layer Edge.Cuts) (width 0.05))
 (gr_line (start 109.5 52.5) (end 112.5 52.5) (layer Edge.Cuts) (width 0.05))
 (gr_line (start 148 50) (end 113.5 50) (layer Edge.Cuts) (width 0.05))
 (gr_arc (start 108.5 50.5) (end 109 50.5) (angle -90) (layer Edge.Cuts) (width 0.05))
 (gr_line (start 150 52) (end 150 98) (layer Edge.Cuts) (width 0.05))
 (segment (start 104.73 92.78) (end 104.73 90.24) (width 0.6) (layer F.Cu) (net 1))
 (segment (start 104.73 90.24) (end 104.73 87.7) (width 0.6) (layer F.Cu) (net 1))
 (segment (start 104.73 57.22) (end 101.124 57.22) (width 0.6) (layer B.Cu) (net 11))
 (segment (start 101.124 57.22) (end 100.762 57.582) (width 0.6) (layer B.Cu) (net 11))
 (segment (start 101.162 62.3) (end 104.73 62.3) (width 0.6) (layer B.Cu) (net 11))
 (segment (start 100.762 61.9) (end 101.162 62.3) (width 0.6) (layer B.Cu) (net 11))
 (segment (start 104.73 59.76) (end 100.908 59.76) (width 0.6) (layer B.Cu) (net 11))
 (segment (start 100.908 59.76) (end 100.762 59.614) (width 0.6) (layer B.Cu) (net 11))
 (segment (start 100.762 59.614) (end 100.762 61.9) (width 0.6) (layer B.Cu) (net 11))
 (segment (start 100.762 57.582) (end 100.762 59.614) (width 0.6) (layer B.Cu) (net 11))
 (segment (start 104.73 57.22) (end 101.124 57.22) (width 0.6) (layer F.Cu) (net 11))
 (segment (start 101.124 57.22) (end 100.762 57.582) (width 0.6) (layer F.Cu) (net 11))
 (segment (start 100.762 57.582) (end 100.762 61.9) (width 0.6) (layer F.Cu) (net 11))
 (segment (start 101.162 62.3) (end 104.73 62.3) (width 0.6) (layer F.Cu) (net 11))
 (segment (start 100.762 61.9) (end 101.162 62.3) (width 0.6) (layer F.Cu) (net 11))
 (segment (start 100.908 59.76) (end 100.762 59.614) (width 0.6) (layer F.Cu) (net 11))
 (segment (start 104.73 59.76) (end 100.908 59.76) (width 0.6) (layer F.Cu) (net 11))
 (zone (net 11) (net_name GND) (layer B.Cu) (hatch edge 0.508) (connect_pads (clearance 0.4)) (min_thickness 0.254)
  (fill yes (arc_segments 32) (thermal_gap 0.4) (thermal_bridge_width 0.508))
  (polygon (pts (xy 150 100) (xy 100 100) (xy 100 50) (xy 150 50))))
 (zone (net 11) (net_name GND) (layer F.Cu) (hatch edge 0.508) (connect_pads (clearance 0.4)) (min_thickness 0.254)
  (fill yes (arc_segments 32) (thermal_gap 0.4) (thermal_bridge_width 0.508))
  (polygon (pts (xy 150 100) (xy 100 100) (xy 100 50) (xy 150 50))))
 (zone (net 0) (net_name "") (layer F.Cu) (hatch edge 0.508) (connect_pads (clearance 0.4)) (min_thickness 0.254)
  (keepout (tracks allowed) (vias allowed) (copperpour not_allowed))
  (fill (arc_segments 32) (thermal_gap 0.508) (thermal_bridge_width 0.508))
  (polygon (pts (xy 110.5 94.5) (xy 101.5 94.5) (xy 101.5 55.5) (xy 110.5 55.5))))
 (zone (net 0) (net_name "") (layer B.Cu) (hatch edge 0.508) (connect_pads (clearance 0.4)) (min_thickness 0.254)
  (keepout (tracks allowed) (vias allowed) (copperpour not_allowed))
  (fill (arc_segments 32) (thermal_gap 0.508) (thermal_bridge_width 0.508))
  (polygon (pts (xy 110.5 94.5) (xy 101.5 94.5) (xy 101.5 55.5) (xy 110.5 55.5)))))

